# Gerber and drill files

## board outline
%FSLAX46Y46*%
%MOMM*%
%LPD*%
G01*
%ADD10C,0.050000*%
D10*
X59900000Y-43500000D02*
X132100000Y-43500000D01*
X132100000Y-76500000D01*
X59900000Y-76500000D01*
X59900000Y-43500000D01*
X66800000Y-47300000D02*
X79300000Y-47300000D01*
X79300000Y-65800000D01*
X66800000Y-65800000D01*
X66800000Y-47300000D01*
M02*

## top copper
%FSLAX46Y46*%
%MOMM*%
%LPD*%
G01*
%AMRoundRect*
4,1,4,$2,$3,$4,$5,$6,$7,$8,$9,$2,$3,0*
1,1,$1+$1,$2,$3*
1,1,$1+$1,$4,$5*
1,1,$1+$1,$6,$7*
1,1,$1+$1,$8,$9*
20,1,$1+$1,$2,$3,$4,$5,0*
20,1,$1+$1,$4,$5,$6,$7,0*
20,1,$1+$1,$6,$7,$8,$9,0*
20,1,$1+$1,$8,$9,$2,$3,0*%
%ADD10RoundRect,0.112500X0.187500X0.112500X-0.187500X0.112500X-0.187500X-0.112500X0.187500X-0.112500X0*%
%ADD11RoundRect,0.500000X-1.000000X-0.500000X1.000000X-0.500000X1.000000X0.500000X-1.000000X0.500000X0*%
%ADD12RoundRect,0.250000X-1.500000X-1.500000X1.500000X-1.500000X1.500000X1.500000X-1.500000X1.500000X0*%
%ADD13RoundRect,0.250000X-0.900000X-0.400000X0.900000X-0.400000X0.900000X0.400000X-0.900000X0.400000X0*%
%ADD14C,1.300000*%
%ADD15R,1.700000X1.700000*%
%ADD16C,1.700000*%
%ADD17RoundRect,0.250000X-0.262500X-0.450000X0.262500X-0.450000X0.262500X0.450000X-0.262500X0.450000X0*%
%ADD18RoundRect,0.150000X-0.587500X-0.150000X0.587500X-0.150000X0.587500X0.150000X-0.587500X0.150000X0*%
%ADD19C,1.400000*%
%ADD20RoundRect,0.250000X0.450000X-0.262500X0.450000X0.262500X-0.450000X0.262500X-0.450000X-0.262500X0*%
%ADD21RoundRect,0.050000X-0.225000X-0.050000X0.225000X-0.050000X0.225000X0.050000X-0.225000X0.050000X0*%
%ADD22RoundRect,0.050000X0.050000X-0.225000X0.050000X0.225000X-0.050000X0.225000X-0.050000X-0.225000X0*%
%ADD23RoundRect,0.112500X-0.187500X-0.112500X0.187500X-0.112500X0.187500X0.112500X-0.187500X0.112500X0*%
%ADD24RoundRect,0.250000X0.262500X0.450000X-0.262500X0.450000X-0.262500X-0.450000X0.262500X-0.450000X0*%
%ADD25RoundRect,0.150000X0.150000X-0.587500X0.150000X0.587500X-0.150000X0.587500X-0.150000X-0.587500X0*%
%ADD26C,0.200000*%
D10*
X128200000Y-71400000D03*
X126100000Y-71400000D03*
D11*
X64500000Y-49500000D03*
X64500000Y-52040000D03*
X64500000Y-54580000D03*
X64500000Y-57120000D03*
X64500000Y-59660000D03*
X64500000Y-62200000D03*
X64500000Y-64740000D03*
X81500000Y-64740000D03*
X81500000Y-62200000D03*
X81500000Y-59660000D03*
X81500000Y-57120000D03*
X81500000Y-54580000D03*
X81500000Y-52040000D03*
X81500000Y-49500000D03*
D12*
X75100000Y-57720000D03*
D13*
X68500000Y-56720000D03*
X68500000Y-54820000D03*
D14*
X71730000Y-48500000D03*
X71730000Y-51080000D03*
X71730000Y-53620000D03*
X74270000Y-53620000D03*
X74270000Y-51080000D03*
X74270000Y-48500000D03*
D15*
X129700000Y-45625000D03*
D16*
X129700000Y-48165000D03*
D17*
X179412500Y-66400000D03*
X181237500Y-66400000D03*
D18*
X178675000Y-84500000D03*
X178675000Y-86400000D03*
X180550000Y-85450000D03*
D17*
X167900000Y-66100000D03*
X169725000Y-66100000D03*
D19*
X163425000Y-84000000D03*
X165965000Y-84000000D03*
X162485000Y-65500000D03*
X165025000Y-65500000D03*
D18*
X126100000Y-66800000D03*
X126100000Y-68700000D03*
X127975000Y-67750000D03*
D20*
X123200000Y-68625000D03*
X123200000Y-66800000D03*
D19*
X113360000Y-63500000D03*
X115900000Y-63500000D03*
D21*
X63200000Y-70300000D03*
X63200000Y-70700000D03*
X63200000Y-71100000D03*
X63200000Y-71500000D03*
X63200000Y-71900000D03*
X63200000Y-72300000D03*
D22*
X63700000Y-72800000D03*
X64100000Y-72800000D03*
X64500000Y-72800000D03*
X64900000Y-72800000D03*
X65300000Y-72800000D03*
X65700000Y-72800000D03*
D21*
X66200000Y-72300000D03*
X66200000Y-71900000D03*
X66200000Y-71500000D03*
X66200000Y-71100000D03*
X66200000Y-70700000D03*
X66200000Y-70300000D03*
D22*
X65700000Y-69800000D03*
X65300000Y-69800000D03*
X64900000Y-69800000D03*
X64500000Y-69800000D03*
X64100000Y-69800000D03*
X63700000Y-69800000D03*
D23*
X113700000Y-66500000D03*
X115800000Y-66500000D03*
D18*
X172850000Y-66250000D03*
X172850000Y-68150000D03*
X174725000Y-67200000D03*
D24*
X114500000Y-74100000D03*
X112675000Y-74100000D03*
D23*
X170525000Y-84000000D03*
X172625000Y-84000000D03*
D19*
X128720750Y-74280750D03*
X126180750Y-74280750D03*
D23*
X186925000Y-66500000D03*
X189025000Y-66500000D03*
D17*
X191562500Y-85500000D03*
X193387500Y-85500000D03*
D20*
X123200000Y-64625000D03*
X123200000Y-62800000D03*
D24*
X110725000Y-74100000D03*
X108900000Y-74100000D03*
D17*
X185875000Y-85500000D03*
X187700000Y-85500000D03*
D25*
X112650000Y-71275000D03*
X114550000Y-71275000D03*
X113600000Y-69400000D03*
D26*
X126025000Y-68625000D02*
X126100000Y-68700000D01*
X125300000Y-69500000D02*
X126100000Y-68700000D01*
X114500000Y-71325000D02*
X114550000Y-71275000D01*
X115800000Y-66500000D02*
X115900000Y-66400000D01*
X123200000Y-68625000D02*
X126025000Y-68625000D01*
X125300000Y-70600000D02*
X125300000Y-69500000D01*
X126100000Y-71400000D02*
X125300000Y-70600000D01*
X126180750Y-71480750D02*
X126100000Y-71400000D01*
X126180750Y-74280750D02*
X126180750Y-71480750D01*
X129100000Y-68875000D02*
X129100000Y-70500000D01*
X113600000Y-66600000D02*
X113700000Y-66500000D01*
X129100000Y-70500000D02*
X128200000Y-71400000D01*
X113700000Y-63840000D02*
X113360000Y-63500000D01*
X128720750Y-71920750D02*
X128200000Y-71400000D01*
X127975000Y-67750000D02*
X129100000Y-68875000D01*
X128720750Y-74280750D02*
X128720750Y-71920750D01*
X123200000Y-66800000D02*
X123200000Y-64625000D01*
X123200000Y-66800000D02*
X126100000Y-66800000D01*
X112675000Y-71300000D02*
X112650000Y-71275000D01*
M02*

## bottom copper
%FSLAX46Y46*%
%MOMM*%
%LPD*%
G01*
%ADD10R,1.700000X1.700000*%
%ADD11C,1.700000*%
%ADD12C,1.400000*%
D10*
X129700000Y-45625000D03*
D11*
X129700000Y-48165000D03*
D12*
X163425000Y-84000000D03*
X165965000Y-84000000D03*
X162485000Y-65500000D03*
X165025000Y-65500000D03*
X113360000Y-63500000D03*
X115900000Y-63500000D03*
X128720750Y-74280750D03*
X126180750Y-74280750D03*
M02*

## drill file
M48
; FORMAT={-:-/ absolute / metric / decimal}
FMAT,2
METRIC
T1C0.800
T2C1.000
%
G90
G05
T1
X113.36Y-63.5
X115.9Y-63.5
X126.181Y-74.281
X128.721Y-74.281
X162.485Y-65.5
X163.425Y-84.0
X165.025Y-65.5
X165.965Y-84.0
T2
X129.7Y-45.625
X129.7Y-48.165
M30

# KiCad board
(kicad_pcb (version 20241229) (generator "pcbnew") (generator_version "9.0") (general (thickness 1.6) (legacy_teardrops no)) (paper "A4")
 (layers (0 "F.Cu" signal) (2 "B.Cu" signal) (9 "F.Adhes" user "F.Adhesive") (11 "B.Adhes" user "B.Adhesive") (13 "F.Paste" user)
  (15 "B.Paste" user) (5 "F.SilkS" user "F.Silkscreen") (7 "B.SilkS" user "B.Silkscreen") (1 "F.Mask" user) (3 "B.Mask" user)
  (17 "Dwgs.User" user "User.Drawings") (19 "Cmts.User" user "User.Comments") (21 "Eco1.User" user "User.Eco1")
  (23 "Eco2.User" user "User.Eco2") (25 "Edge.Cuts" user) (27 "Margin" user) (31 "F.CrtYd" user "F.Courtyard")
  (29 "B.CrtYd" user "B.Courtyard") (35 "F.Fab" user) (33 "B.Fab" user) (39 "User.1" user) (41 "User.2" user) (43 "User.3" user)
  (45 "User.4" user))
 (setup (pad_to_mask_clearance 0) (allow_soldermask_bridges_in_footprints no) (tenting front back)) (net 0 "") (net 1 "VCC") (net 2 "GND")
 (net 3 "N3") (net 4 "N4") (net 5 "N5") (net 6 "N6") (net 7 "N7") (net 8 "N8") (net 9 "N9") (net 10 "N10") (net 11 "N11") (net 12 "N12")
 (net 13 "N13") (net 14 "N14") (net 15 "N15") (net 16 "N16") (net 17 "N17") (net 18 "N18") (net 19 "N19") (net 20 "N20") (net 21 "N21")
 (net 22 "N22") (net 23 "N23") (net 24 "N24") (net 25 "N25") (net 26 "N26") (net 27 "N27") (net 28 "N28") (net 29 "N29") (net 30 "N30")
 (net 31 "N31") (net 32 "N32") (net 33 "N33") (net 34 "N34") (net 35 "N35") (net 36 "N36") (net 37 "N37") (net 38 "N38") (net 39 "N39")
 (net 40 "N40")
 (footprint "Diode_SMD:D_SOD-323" (layer "F.Cu") (at 127.15 71.4 180)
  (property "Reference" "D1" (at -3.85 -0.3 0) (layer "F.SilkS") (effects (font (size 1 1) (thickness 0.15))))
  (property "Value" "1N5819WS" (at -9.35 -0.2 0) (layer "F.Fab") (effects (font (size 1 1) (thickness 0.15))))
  (pad "1" smd roundrect (at -1.05 0 180) (size 0.6 0.45) (layers "F.Cu" "F.Mask" "F.Paste") (roundrect_rratio 0.25) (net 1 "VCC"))
  (pad "2" smd roundrect (at 1.05 0 180) (size 0.6 0.45) (layers "F.Cu" "F.Mask" "F.Paste") (roundrect_rratio 0.25) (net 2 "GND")))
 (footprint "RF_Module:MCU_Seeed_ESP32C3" (layer "F.Cu") (at 73 57.12)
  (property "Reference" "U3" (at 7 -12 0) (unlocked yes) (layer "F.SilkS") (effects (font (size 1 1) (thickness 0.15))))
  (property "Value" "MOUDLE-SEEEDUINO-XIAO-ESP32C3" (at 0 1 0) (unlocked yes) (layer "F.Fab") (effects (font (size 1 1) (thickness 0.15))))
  (pad "" smd roundrect (at 1.1 -0.4) (size 1.5 1.5) (layers "F.Paste") (roundrect_rratio 0.1666666667))
  (pad "" smd roundrect (at 1.1 1.6) (size 1.5 1.5) (layers "F.Paste") (roundrect_rratio 0.1666666667))
  (pad "" smd roundrect (at 3.1 -0.4) (size 1.5 1.5) (layers "F.Paste") (roundrect_rratio 0.1666666667))
  (pad "" smd roundrect (at 3.1 1.6) (size 1.5 1.5) (layers "F.Paste") (roundrect_rratio 0.1666666667))
  (pad "1" smd roundrect (at -8.5 -7.62) (size 3 2) (layers "F.Cu" "F.Mask" "F.Paste") (roundrect_rratio 0.25) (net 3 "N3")
   (thermal_bridge_angle 45))
  (pad "2" smd roundrect (at -8.5 -5.08) (size 3 2) (layers "F.Cu" "F.Mask" "F.Paste") (roundrect_rratio 0.25) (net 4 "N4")
   (thermal_bridge_angle 45))
  (pad "3" smd roundrect (at -8.5 -2.54) (size 3 2) (layers "F.Cu" "F.Mask" "F.Paste") (roundrect_rratio 0.25) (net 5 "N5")
   (thermal_bridge_angle 45))
  (pad "4" smd roundrect (at -8.5 0) (size 3 2) (layers "F.Cu" "F.Mask" "F.Paste") (roundrect_rratio 0.25) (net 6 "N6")
   (thermal_bridge_angle 45))
  (pad "5" smd roundrect (at -8.5 2.54) (size 3 2) (layers "F.Cu" "F.Mask" "F.Paste") (roundrect_rratio 0.25) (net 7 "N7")
   (thermal_bridge_angle 45))
  (pad "6" smd roundrect (at -8.5 5.08) (size 3 2) (layers "F.Cu" "F.Mask" "F.Paste") (roundrect_rratio 0.25) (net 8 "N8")
   (thermal_bridge_angle 45))
  (pad "7" smd roundrect (at -8.5 7.62) (size 3 2) (layers "F.Cu" "F.Mask" "F.Paste") (roundrect_rratio 0.25) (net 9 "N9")
   (thermal_bridge_angle 45))
  (pad "8" smd roundrect (at 8.5 7.62) (size 3 2) (layers "F.Cu" "F.Mask" "F.Paste") (roundrect_rratio 0.25) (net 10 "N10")
   (thermal_bridge_angle 45))
  (pad "9" smd roundrect (at 8.5 5.08) (size 3 2) (layers "F.Cu" "F.Mask" "F.Paste") (roundrect_rratio 0.25) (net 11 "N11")
   (thermal_bridge_angle 45))
  (pad "10" smd roundrect (at 8.5 2.54) (size 3 2) (layers "F.Cu" "F.Mask" "F.Paste") (roundrect_rratio 0.25) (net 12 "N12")
   (thermal_bridge_angle 45))
  (pad "11" smd roundrect (at 8.5 0) (size 3 2) (layers "F.Cu" "F.Mask" "F.Paste") (roundrect_rratio 0.25) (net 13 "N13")
   (thermal_bridge_angle 45))
  (pad "12" smd roundrect (at 8.5 -2.54) (size 3 2) (layers "F.Cu" "F.Mask" "F.Paste") (roundrect_rratio 0.25) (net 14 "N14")
   (thermal_bridge_angle 45))
  (pad "13" smd roundrect (at 8.5 -5.08) (size 3 2) (layers "F.Cu" "F.Mask" "F.Paste") (roundrect_rratio 0.25) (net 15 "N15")
   (thermal_bridge_angle 45))
  (pad "14" smd roundrect (at 8.5 -7.62) (size 3 2) (layers "F.Cu" "F.Mask" "F.Paste") (roundrect_rratio 0.25) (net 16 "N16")
   (thermal_bridge_angle 45))
  (pad "15" smd roundrect (at 2.1 0.6) (size 3.5 3.5) (layers "F.Cu" "F.Mask") (roundrect_rratio 0.07142857143))
  (pad "16" smd roundrect (at -4.5 -0.4) (size 2.3 1.3) (layers "F.Cu" "F.Mask" "F.Paste") (roundrect_rratio 0.1923076923))
  (pad "17" smd roundrect (at -4.5 -2.3) (size 2.3 1.3) (layers "F.Cu" "F.Mask" "F.Paste") (roundrect_rratio 0.1923076923))
  (pad "18" smd circle (at -1.27 -8.62) (size 1.3 1.3) (layers "F.Cu" "F.Mask" "F.Paste"))
  (pad "19" smd circle (at -1.27 -6.04) (size 1.3 1.3) (layers "F.Cu" "F.Mask" "F.Paste"))
  (pad "20" smd circle (at -1.27 -3.5) (size 1.3 1.3) (layers "F.Cu" "F.Mask" "F.Paste"))
  (pad "21" smd circle (at 1.27 -3.5) (size 1.3 1.3) (layers "F.Cu" "F.Mask" "F.Paste"))
  (pad "22" smd circle (at 1.27 -6.04) (size 1.3 1.3) (layers "F.Cu" "F.Mask" "F.Paste"))
  (pad "23" smd circle (at 1.27 -8.62) (size 1.3 1.3) (layers "F.Cu" "F.Mask" "F.Paste")))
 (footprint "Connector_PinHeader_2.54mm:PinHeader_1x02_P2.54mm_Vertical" (layer "F.Cu") (at 129.7 45.625)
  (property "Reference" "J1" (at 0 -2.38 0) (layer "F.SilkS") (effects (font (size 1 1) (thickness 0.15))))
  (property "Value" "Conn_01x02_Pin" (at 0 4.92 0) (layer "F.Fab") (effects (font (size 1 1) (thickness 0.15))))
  (pad "1" thru_hole rect (at 0 0) (size 1.7 1.7) (drill 1) (layers "*.Cu" "*.Mask") (remove_unused_layers no) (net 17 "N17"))
  (pad "2" thru_hole circle (at 0 2.54) (size 1.7 1.7) (drill 1) (layers "*.Cu" "*.Mask") (remove_unused_layers no) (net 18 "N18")))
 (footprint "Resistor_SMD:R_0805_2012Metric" (layer "F.Cu") (at 180.325 66.4)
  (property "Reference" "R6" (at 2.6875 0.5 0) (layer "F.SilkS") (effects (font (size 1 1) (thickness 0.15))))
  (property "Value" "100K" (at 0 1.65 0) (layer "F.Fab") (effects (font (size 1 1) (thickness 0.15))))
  (pad "1" smd roundrect (at -0.9125 0) (size 1.025 1.4) (layers "F.Cu" "F.Mask" "F.Paste") (roundrect_rratio 0.243902) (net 2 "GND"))
  (pad "2" smd roundrect (at 0.9125 0) (size 1.025 1.4) (layers "F.Cu" "F.Mask" "F.Paste") (roundrect_rratio 0.243902) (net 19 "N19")))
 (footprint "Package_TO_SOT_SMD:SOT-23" (layer "F.Cu") (at 179.6125 85.45)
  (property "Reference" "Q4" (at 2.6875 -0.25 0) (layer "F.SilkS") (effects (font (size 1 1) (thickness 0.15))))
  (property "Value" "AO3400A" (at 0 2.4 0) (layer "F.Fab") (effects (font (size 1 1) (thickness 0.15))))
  (pad "1" smd roundrect (at -0.9375 -0.95) (size 1.475 0.6) (layers "F.Cu" "F.Mask" "F.Paste") (roundrect_rratio 0.25) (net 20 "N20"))
  (pad "2" smd roundrect (at -0.9375 0.95) (size 1.475 0.6) (layers "F.Cu" "F.Mask" "F.Paste") (roundrect_rratio 0.25) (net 2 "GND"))
  (pad "3" smd roundrect (at 0.9375 0) (size 1.475 0.6) (layers "F.Cu" "F.Mask" "F.Paste") (roundrect_rratio 0.25) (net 1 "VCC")))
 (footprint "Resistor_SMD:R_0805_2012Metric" (layer "F.Cu") (at 168.8125 66.1)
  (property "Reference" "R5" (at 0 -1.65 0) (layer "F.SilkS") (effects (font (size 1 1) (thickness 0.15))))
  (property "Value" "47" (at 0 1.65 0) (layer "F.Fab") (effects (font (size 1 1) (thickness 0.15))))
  (pad "1" smd roundrect (at -0.9125 0) (size 1.025 1.4) (layers "F.Cu" "F.Mask" "F.Paste") (roundrect_rratio 0.243902) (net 19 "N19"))
  (pad "2" smd roundrect (at 0.9125 0) (size 1.025 1.4) (layers "F.Cu" "F.Mask" "F.Paste") (roundrect_rratio 0.243902) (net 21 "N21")))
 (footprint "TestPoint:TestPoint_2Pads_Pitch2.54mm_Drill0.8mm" (layer "F.Cu") (at 163.425 84)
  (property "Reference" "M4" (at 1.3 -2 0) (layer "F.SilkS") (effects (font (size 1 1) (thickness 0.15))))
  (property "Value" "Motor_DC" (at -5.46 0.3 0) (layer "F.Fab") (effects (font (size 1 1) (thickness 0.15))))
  (pad "1" thru_hole circle (at 0 0) (size 1.4 1.4) (drill 0.8) (layers "*.Cu" "*.Mask") (remove_unused_layers no) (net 1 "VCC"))
  (pad "2" thru_hole circle (at 2.54 0) (size 1.4 1.4) (drill 0.8) (layers "*.Cu" "*.Mask") (remove_unused_layers no) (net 2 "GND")))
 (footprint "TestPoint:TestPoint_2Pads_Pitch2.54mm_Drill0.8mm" (layer "F.Cu") (at 162.485 65.5)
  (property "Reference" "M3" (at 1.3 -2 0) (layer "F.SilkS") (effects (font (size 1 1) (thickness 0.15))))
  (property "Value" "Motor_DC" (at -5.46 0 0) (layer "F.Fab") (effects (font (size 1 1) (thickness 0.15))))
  (pad "1" thru_hole circle (at 0 0) (size 1.4 1.4) (drill 0.8) (layers "*.Cu" "*.Mask") (remove_unused_layers no) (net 1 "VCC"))
  (pad "2" thru_hole circle (at 2.54 0) (size 1.4 1.4) (drill 0.8) (layers "*.Cu" "*.Mask") (remove_unused_layers no) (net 2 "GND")))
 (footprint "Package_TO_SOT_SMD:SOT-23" (layer "F.Cu") (at 127.0375 67.75)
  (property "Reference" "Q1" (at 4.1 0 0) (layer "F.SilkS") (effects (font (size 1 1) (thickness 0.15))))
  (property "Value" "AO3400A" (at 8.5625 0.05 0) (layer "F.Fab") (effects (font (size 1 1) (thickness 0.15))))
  (pad "1" smd roundrect (at -0.9375 -0.95) (size 1.475 0.6) (layers "F.Cu" "F.Mask" "F.Paste") (roundrect_rratio 0.25) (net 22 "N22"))
  (pad "2" smd roundrect (at -0.9375 0.95) (size 1.475 0.6) (layers "F.Cu" "F.Mask" "F.Paste") (roundrect_rratio 0.25) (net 2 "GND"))
  (pad "3" smd roundrect (at 0.9375 0) (size 1.475 0.6) (layers "F.Cu" "F.Mask" "F.Paste") (roundrect_rratio 0.25) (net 1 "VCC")))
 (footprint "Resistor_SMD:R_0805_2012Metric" (layer "F.Cu") (at 123.2 67.7125 90)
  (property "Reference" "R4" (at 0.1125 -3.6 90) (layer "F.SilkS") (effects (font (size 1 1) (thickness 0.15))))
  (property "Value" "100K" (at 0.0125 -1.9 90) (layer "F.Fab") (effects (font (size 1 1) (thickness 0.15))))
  (pad "1" smd roundrect (at -0.9125 0 90) (size 1.025 1.4) (layers "F.Cu" "F.Mask" "F.Paste") (roundrect_rratio 0.243902) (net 2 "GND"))
  (pad "2" smd roundrect (at 0.9125 0 90) (size 1.025 1.4) (layers "F.Cu" "F.Mask" "F.Paste") (roundrect_rratio 0.243902) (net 22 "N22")))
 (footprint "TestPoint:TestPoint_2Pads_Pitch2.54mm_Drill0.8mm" (layer "F.Cu") (at 113.36 63.5)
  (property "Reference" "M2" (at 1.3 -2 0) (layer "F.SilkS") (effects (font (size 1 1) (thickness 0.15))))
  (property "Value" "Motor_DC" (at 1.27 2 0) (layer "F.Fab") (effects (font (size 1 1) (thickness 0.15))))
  (pad "1" thru_hole circle (at 0 0) (size 1.4 1.4) (drill 0.8) (layers "*.Cu" "*.Mask") (remove_unused_layers no) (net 1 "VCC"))
  (pad "2" thru_hole circle (at 2.54 0) (size 1.4 1.4) (drill 0.8) (layers "*.Cu" "*.Mask") (remove_unused_layers no) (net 2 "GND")))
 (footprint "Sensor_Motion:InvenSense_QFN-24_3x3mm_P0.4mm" (layer "F.Cu") (at 64.7 71.3)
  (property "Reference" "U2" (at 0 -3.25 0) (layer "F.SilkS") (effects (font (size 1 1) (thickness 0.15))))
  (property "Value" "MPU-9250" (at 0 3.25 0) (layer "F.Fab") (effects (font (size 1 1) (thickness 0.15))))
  (pad "1" smd roundrect (at -1.5 -1) (size 0.55 0.2) (layers "F.Cu" "F.Mask" "F.Paste") (roundrect_rratio 0.25) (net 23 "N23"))
  (pad "2" smd roundrect (at -1.5 -0.6) (size 0.55 0.2) (layers "F.Cu" "F.Mask" "F.Paste") (roundrect_rratio 0.25))
  (pad "3" smd roundrect (at -1.5 -0.2) (size 0.55 0.2) (layers "F.Cu" "F.Mask" "F.Paste") (roundrect_rratio 0.25))
  (pad "4" smd roundrect (at -1.5 0.2) (size 0.55 0.2) (layers "F.Cu" "F.Mask" "F.Paste") (roundrect_rratio 0.25))
  (pad "5" smd roundrect (at -1.5 0.6) (size 0.55 0.2) (layers "F.Cu" "F.Mask" "F.Paste") (roundrect_rratio 0.25))
  (pad "6" smd roundrect (at -1.5 1) (size 0.55 0.2) (layers "F.Cu" "F.Mask" "F.Paste") (roundrect_rratio 0.25))
  (pad "7" smd roundrect (at -1 1.5 90) (size 0.55 0.2) (layers "F.Cu" "F.Mask" "F.Paste") (roundrect_rratio 0.25) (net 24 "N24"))
  (pad "8" smd roundrect (at -0.6 1.5 90) (size 0.55 0.2) (layers "F.Cu" "F.Mask" "F.Paste") (roundrect_rratio 0.25) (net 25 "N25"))
  (pad "9" smd roundrect (at -0.2 1.5 90) (size 0.55 0.2) (layers "F.Cu" "F.Mask" "F.Paste") (roundrect_rratio 0.25) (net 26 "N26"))
  (pad "10" smd roundrect (at 0.2 1.5 90) (size 0.55 0.2) (layers "F.Cu" "F.Mask" "F.Paste") (roundrect_rratio 0.25) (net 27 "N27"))
  (pad "11" smd roundrect (at 0.6 1.5 90) (size 0.55 0.2) (layers "F.Cu" "F.Mask" "F.Paste") (roundrect_rratio 0.25) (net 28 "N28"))
  (pad "12" smd roundrect (at 1 1.5 90) (size 0.55 0.2) (layers "F.Cu" "F.Mask" "F.Paste") (roundrect_rratio 0.25) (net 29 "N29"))
  (pad "13" smd roundrect (at 1.5 1) (size 0.55 0.2) (layers "F.Cu" "F.Mask" "F.Paste") (roundrect_rratio 0.25) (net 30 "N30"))
  (pad "14" smd roundrect (at 1.5 0.6) (size 0.55 0.2) (layers "F.Cu" "F.Mask" "F.Paste") (roundrect_rratio 0.25))
  (pad "15" smd roundrect (at 1.5 0.2) (size 0.55 0.2) (layers "F.Cu" "F.Mask" "F.Paste") (roundrect_rratio 0.25))
  (pad "16" smd roundrect (at 1.5 -0.2) (size 0.55 0.2) (layers "F.Cu" "F.Mask" "F.Paste") (roundrect_rratio 0.25))
  (pad "17" smd roundrect (at 1.5 -0.6) (size 0.55 0.2) (layers "F.Cu" "F.Mask" "F.Paste") (roundrect_rratio 0.25))
  (pad "18" smd roundrect (at 1.5 -1) (size 0.55 0.2) (layers "F.Cu" "F.Mask" "F.Paste") (roundrect_rratio 0.25) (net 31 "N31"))
  (pad "19" smd roundrect (at 1 -1.5 90) (size 0.55 0.2) (layers "F.Cu" "F.Mask" "F.Paste") (roundrect_rratio 0.25))
  (pad "20" smd roundrect (at 0.6 -1.5 90) (size 0.55 0.2) (layers "F.Cu" "F.Mask" "F.Paste") (roundrect_rratio 0.25) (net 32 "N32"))
  (pad "21" smd roundrect (at 0.2 -1.5 90) (size 0.55 0.2) (layers "F.Cu" "F.Mask" "F.Paste") (roundrect_rratio 0.25) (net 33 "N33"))
  (pad "22" smd roundrect (at -0.2 -1.5 90) (size 0.55 0.2) (layers "F.Cu" "F.Mask" "F.Paste") (roundrect_rratio 0.25) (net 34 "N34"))
  (pad "23" smd roundrect (at -0.6 -1.5 90) (size 0.55 0.2) (layers "F.Cu" "F.Mask" "F.Paste") (roundrect_rratio 0.25) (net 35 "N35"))
  (pad "24" smd roundrect (at -1 -1.5 90) (size 0.55 0.2) (layers "F.Cu" "F.Mask" "F.Paste") (roundrect_rratio 0.25) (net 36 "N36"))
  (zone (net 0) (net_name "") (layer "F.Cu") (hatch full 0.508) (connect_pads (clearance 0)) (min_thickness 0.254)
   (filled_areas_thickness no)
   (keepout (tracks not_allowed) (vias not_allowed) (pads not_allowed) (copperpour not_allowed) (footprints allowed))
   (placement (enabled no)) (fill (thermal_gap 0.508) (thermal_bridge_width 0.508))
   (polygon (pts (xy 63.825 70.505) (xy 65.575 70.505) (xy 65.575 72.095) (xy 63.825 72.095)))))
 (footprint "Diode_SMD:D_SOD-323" (layer "F.Cu") (at 114.75 66.5)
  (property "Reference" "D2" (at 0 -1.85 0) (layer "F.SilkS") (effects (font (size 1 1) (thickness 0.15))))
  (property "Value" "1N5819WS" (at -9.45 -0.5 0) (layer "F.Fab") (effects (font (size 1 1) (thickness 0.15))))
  (pad "1" smd roundrect (at -1.05 0) (size 0.6 0.45) (layers "F.Cu" "F.Mask" "F.Paste") (roundrect_rratio 0.25) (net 1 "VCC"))
  (pad "2" smd roundrect (at 1.05 0) (size 0.6 0.45) (layers "F.Cu" "F.Mask" "F.Paste") (roundrect_rratio 0.25) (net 2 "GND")))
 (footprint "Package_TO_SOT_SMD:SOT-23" (layer "F.Cu") (at 173.7875 67.2)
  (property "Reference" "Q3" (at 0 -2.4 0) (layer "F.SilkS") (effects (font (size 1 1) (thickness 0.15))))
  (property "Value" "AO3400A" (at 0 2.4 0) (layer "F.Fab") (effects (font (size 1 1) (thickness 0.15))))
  (pad "1" smd roundrect (at -0.9375 -0.95) (size 1.475 0.6) (layers "F.Cu" "F.Mask" "F.Paste") (roundrect_rratio 0.25) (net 19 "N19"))
  (pad "2" smd roundrect (at -0.9375 0.95) (size 1.475 0.6) (layers "F.Cu" "F.Mask" "F.Paste") (roundrect_rratio 0.25) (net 2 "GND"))
  (pad "3" smd roundrect (at 0.9375 0) (size 1.475 0.6) (layers "F.Cu" "F.Mask" "F.Paste") (roundrect_rratio 0.25) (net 1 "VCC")))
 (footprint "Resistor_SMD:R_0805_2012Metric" (layer "F.Cu") (at 113.5875 74.1 180)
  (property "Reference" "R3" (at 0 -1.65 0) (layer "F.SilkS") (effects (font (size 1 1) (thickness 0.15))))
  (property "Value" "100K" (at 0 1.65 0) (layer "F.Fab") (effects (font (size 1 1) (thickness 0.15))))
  (pad "1" smd roundrect (at -0.9125 0 180) (size 1.025 1.4) (layers "F.Cu" "F.Mask" "F.Paste") (roundrect_rratio 0.243902) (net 2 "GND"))
  (pad "2" smd roundrect (at 0.9125 0 180) (size 1.025 1.4) (layers "F.Cu" "F.Mask" "F.Paste") (roundrect_rratio 0.243902) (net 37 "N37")))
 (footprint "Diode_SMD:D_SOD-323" (layer "F.Cu") (at 171.575 84)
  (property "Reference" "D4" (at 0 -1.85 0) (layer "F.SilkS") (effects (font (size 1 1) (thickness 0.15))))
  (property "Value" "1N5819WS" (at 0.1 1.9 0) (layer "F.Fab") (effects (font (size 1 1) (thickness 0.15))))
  (pad "1" smd roundrect (at -1.05 0) (size 0.6 0.45) (layers "F.Cu" "F.Mask" "F.Paste") (roundrect_rratio 0.25) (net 1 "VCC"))
  (pad "2" smd roundrect (at 1.05 0) (size 0.6 0.45) (layers "F.Cu" "F.Mask" "F.Paste") (roundrect_rratio 0.25) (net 2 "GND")))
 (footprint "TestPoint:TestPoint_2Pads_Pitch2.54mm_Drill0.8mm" (layer "F.Cu") (at 128.72075 74.28075 180)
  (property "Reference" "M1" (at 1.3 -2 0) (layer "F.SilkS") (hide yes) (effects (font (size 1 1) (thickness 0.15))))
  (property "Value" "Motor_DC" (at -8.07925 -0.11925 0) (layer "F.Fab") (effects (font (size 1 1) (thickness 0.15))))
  (pad "1" thru_hole circle (at 0 0 180) (size 1.4 1.4) (drill 0.8) (layers "*.Cu" "*.Mask") (remove_unused_layers no) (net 1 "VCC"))
  (pad "2" thru_hole circle (at 2.54 0 180) (size 1.4 1.4) (drill 0.8) (layers "*.Cu" "*.Mask") (remove_unused_layers no) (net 2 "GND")))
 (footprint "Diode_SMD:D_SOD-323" (layer "F.Cu") (at 187.975 66.5)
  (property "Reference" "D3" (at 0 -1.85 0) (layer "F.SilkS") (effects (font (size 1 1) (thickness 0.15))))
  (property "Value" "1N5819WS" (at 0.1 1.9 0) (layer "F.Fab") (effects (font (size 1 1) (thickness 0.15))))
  (pad "1" smd roundrect (at -1.05 0) (size 0.6 0.45) (layers "F.Cu" "F.Mask" "F.Paste") (roundrect_rratio 0.25) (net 1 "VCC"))
  (pad "2" smd roundrect (at 1.05 0) (size 0.6 0.45) (layers "F.Cu" "F.Mask" "F.Paste") (roundrect_rratio 0.25) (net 2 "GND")))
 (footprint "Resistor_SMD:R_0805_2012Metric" (layer "F.Cu") (at 192.475 85.5)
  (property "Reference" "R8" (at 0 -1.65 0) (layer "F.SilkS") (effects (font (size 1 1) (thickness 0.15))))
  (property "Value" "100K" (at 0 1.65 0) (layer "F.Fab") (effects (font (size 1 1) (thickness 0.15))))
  (pad "1" smd roundrect (at -0.9125 0) (size 1.025 1.4) (layers "F.Cu" "F.Mask" "F.Paste") (roundrect_rratio 0.243902) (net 2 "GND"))
  (pad "2" smd roundrect (at 0.9125 0) (size 1.025 1.4) (layers "F.Cu" "F.Mask" "F.Paste") (roundrect_rratio 0.243902) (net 20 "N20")))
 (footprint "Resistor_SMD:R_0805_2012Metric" (layer "F.Cu") (at 123.2 63.7125 90)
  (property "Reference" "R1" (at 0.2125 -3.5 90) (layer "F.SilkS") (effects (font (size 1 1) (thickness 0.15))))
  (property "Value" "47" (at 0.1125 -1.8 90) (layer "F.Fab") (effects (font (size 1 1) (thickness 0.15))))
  (pad "1" smd roundrect (at -0.9125 0 90) (size 1.025 1.4) (layers "F.Cu" "F.Mask" "F.Paste") (roundrect_rratio 0.243902) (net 22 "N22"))
  (pad "2" smd roundrect (at 0.9125 0 90) (size 1.025 1.4) (layers "F.Cu" "F.Mask" "F.Paste") (roundrect_rratio 0.243902) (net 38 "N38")))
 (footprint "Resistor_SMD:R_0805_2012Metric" (layer "F.Cu") (at 109.8125 74.1 180)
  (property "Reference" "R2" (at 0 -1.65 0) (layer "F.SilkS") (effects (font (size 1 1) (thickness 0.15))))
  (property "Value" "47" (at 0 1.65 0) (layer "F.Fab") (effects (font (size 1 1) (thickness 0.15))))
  (pad "1" smd roundrect (at -0.9125 0 180) (size 1.025 1.4) (layers "F.Cu" "F.Mask" "F.Paste") (roundrect_rratio 0.243902) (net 37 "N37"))
  (pad "2" smd roundrect (at 0.9125 0 180) (size 1.025 1.4) (layers "F.Cu" "F.Mask" "F.Paste") (roundrect_rratio 0.243902) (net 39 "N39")))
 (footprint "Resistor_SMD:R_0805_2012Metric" (layer "F.Cu") (at 186.7875 85.5)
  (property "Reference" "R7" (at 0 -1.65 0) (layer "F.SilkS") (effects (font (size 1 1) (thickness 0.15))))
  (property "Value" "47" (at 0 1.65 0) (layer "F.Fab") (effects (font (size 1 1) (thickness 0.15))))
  (pad "1" smd roundrect (at -0.9125 0) (size 1.025 1.4) (layers "F.Cu" "F.Mask" "F.Paste") (roundrect_rratio 0.243902) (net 20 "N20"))
  (pad "2" smd roundrect (at 0.9125 0) (size 1.025 1.4) (layers "F.Cu" "F.Mask" "F.Paste") (roundrect_rratio 0.243902) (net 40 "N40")))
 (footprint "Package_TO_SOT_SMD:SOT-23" (layer "F.Cu") (at 113.6 70.3375 90)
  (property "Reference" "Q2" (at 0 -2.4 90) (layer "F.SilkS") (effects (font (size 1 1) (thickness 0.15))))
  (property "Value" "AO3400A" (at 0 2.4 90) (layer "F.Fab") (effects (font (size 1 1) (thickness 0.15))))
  (pad "1" smd roundrect (at -0.9375 -0.95 90) (size 1.475 0.6) (layers "F.Cu" "F.Mask" "F.Paste") (roundrect_rratio 0.25) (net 37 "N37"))
  (pad "2" smd roundrect (at -0.9375 0.95 90) (size 1.475 0.6) (layers "F.Cu" "F.Mask" "F.Paste") (roundrect_rratio 0.25) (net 2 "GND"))
  (pad "3" smd roundrect (at 0.9375 0 90) (size 1.475 0.6) (layers "F.Cu" "F.Mask" "F.Paste") (roundrect_rratio 0.25) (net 1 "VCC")))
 (gr_rect (start 59.9 43.5) (end 132.1 76.5) (stroke (width 0.05) (type default)) (fill no) (layer "Edge.Cuts"))
 (gr_rect (start 66.8 47.3) (end 79.3 65.8) (stroke (width 0.05) (type default)) (fill no) (layer "Edge.Cuts"))
 (segment (start 126.025 68.625) (end 126.1 68.7) (width 0.2) (layer "F.Cu") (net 2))
 (segment (start 125.3 69.5) (end 126.1 68.7) (width 0.2) (layer "F.Cu") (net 2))
 (segment (start 114.5 71.325) (end 114.55 71.275) (width 0.2) (layer "F.Cu") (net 2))
 (segment (start 115.8 66.5) (end 115.9 66.4) (width 0.2) (layer "F.Cu") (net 2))
 (segment (start 123.2 68.625) (end 126.025 68.625) (width 0.2) (layer "F.Cu") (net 2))
 (segment (start 125.3 70.6) (end 125.3 69.5) (width 0.2) (layer "F.Cu") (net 2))
 (segment (start 126.1 71.4) (end 125.3 70.6) (width 0.2) (layer "F.Cu") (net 2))
 (segment (start 126.18075 71.48075) (end 126.1 71.4) (width 0.2) (layer "F.Cu") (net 2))
 (segment (start 126.18075 74.28075) (end 126.18075 71.48075) (width 0.2) (layer "F.Cu") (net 2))
 (segment (start 129.1 68.875) (end 129.1 70.5) (width 0.2) (layer "F.Cu") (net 1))
 (segment (start 113.6 66.6) (end 113.7 66.5) (width 0.2) (layer "F.Cu") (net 1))
 (segment (start 129.1 70.5) (end 128.2 71.4) (width 0.2) (layer "F.Cu") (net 1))
 (segment (start 113.7 63.84) (end 113.36 63.5) (width 0.2) (layer "F.Cu") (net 1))
 (segment (start 128.72075 71.92075) (end 128.2 71.4) (width 0.2) (layer "F.Cu") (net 1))
 (segment (start 127.975 67.75) (end 129.1 68.875) (width 0.2) (layer "F.Cu") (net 1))
 (segment (start 128.72075 74.28075) (end 128.72075 71.92075) (width 0.2) (layer "F.Cu") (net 1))
 (segment (start 123.2 66.8) (end 123.2 64.625) (width 0.2) (layer "F.Cu") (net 22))
 (segment (start 123.2 66.8) (end 126.1 66.8) (width 0.2) (layer "F.Cu") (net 22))
 (segment (start 112.675 71.3) (end 112.65 71.275) (width 0.2) (layer "F.Cu") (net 37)))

